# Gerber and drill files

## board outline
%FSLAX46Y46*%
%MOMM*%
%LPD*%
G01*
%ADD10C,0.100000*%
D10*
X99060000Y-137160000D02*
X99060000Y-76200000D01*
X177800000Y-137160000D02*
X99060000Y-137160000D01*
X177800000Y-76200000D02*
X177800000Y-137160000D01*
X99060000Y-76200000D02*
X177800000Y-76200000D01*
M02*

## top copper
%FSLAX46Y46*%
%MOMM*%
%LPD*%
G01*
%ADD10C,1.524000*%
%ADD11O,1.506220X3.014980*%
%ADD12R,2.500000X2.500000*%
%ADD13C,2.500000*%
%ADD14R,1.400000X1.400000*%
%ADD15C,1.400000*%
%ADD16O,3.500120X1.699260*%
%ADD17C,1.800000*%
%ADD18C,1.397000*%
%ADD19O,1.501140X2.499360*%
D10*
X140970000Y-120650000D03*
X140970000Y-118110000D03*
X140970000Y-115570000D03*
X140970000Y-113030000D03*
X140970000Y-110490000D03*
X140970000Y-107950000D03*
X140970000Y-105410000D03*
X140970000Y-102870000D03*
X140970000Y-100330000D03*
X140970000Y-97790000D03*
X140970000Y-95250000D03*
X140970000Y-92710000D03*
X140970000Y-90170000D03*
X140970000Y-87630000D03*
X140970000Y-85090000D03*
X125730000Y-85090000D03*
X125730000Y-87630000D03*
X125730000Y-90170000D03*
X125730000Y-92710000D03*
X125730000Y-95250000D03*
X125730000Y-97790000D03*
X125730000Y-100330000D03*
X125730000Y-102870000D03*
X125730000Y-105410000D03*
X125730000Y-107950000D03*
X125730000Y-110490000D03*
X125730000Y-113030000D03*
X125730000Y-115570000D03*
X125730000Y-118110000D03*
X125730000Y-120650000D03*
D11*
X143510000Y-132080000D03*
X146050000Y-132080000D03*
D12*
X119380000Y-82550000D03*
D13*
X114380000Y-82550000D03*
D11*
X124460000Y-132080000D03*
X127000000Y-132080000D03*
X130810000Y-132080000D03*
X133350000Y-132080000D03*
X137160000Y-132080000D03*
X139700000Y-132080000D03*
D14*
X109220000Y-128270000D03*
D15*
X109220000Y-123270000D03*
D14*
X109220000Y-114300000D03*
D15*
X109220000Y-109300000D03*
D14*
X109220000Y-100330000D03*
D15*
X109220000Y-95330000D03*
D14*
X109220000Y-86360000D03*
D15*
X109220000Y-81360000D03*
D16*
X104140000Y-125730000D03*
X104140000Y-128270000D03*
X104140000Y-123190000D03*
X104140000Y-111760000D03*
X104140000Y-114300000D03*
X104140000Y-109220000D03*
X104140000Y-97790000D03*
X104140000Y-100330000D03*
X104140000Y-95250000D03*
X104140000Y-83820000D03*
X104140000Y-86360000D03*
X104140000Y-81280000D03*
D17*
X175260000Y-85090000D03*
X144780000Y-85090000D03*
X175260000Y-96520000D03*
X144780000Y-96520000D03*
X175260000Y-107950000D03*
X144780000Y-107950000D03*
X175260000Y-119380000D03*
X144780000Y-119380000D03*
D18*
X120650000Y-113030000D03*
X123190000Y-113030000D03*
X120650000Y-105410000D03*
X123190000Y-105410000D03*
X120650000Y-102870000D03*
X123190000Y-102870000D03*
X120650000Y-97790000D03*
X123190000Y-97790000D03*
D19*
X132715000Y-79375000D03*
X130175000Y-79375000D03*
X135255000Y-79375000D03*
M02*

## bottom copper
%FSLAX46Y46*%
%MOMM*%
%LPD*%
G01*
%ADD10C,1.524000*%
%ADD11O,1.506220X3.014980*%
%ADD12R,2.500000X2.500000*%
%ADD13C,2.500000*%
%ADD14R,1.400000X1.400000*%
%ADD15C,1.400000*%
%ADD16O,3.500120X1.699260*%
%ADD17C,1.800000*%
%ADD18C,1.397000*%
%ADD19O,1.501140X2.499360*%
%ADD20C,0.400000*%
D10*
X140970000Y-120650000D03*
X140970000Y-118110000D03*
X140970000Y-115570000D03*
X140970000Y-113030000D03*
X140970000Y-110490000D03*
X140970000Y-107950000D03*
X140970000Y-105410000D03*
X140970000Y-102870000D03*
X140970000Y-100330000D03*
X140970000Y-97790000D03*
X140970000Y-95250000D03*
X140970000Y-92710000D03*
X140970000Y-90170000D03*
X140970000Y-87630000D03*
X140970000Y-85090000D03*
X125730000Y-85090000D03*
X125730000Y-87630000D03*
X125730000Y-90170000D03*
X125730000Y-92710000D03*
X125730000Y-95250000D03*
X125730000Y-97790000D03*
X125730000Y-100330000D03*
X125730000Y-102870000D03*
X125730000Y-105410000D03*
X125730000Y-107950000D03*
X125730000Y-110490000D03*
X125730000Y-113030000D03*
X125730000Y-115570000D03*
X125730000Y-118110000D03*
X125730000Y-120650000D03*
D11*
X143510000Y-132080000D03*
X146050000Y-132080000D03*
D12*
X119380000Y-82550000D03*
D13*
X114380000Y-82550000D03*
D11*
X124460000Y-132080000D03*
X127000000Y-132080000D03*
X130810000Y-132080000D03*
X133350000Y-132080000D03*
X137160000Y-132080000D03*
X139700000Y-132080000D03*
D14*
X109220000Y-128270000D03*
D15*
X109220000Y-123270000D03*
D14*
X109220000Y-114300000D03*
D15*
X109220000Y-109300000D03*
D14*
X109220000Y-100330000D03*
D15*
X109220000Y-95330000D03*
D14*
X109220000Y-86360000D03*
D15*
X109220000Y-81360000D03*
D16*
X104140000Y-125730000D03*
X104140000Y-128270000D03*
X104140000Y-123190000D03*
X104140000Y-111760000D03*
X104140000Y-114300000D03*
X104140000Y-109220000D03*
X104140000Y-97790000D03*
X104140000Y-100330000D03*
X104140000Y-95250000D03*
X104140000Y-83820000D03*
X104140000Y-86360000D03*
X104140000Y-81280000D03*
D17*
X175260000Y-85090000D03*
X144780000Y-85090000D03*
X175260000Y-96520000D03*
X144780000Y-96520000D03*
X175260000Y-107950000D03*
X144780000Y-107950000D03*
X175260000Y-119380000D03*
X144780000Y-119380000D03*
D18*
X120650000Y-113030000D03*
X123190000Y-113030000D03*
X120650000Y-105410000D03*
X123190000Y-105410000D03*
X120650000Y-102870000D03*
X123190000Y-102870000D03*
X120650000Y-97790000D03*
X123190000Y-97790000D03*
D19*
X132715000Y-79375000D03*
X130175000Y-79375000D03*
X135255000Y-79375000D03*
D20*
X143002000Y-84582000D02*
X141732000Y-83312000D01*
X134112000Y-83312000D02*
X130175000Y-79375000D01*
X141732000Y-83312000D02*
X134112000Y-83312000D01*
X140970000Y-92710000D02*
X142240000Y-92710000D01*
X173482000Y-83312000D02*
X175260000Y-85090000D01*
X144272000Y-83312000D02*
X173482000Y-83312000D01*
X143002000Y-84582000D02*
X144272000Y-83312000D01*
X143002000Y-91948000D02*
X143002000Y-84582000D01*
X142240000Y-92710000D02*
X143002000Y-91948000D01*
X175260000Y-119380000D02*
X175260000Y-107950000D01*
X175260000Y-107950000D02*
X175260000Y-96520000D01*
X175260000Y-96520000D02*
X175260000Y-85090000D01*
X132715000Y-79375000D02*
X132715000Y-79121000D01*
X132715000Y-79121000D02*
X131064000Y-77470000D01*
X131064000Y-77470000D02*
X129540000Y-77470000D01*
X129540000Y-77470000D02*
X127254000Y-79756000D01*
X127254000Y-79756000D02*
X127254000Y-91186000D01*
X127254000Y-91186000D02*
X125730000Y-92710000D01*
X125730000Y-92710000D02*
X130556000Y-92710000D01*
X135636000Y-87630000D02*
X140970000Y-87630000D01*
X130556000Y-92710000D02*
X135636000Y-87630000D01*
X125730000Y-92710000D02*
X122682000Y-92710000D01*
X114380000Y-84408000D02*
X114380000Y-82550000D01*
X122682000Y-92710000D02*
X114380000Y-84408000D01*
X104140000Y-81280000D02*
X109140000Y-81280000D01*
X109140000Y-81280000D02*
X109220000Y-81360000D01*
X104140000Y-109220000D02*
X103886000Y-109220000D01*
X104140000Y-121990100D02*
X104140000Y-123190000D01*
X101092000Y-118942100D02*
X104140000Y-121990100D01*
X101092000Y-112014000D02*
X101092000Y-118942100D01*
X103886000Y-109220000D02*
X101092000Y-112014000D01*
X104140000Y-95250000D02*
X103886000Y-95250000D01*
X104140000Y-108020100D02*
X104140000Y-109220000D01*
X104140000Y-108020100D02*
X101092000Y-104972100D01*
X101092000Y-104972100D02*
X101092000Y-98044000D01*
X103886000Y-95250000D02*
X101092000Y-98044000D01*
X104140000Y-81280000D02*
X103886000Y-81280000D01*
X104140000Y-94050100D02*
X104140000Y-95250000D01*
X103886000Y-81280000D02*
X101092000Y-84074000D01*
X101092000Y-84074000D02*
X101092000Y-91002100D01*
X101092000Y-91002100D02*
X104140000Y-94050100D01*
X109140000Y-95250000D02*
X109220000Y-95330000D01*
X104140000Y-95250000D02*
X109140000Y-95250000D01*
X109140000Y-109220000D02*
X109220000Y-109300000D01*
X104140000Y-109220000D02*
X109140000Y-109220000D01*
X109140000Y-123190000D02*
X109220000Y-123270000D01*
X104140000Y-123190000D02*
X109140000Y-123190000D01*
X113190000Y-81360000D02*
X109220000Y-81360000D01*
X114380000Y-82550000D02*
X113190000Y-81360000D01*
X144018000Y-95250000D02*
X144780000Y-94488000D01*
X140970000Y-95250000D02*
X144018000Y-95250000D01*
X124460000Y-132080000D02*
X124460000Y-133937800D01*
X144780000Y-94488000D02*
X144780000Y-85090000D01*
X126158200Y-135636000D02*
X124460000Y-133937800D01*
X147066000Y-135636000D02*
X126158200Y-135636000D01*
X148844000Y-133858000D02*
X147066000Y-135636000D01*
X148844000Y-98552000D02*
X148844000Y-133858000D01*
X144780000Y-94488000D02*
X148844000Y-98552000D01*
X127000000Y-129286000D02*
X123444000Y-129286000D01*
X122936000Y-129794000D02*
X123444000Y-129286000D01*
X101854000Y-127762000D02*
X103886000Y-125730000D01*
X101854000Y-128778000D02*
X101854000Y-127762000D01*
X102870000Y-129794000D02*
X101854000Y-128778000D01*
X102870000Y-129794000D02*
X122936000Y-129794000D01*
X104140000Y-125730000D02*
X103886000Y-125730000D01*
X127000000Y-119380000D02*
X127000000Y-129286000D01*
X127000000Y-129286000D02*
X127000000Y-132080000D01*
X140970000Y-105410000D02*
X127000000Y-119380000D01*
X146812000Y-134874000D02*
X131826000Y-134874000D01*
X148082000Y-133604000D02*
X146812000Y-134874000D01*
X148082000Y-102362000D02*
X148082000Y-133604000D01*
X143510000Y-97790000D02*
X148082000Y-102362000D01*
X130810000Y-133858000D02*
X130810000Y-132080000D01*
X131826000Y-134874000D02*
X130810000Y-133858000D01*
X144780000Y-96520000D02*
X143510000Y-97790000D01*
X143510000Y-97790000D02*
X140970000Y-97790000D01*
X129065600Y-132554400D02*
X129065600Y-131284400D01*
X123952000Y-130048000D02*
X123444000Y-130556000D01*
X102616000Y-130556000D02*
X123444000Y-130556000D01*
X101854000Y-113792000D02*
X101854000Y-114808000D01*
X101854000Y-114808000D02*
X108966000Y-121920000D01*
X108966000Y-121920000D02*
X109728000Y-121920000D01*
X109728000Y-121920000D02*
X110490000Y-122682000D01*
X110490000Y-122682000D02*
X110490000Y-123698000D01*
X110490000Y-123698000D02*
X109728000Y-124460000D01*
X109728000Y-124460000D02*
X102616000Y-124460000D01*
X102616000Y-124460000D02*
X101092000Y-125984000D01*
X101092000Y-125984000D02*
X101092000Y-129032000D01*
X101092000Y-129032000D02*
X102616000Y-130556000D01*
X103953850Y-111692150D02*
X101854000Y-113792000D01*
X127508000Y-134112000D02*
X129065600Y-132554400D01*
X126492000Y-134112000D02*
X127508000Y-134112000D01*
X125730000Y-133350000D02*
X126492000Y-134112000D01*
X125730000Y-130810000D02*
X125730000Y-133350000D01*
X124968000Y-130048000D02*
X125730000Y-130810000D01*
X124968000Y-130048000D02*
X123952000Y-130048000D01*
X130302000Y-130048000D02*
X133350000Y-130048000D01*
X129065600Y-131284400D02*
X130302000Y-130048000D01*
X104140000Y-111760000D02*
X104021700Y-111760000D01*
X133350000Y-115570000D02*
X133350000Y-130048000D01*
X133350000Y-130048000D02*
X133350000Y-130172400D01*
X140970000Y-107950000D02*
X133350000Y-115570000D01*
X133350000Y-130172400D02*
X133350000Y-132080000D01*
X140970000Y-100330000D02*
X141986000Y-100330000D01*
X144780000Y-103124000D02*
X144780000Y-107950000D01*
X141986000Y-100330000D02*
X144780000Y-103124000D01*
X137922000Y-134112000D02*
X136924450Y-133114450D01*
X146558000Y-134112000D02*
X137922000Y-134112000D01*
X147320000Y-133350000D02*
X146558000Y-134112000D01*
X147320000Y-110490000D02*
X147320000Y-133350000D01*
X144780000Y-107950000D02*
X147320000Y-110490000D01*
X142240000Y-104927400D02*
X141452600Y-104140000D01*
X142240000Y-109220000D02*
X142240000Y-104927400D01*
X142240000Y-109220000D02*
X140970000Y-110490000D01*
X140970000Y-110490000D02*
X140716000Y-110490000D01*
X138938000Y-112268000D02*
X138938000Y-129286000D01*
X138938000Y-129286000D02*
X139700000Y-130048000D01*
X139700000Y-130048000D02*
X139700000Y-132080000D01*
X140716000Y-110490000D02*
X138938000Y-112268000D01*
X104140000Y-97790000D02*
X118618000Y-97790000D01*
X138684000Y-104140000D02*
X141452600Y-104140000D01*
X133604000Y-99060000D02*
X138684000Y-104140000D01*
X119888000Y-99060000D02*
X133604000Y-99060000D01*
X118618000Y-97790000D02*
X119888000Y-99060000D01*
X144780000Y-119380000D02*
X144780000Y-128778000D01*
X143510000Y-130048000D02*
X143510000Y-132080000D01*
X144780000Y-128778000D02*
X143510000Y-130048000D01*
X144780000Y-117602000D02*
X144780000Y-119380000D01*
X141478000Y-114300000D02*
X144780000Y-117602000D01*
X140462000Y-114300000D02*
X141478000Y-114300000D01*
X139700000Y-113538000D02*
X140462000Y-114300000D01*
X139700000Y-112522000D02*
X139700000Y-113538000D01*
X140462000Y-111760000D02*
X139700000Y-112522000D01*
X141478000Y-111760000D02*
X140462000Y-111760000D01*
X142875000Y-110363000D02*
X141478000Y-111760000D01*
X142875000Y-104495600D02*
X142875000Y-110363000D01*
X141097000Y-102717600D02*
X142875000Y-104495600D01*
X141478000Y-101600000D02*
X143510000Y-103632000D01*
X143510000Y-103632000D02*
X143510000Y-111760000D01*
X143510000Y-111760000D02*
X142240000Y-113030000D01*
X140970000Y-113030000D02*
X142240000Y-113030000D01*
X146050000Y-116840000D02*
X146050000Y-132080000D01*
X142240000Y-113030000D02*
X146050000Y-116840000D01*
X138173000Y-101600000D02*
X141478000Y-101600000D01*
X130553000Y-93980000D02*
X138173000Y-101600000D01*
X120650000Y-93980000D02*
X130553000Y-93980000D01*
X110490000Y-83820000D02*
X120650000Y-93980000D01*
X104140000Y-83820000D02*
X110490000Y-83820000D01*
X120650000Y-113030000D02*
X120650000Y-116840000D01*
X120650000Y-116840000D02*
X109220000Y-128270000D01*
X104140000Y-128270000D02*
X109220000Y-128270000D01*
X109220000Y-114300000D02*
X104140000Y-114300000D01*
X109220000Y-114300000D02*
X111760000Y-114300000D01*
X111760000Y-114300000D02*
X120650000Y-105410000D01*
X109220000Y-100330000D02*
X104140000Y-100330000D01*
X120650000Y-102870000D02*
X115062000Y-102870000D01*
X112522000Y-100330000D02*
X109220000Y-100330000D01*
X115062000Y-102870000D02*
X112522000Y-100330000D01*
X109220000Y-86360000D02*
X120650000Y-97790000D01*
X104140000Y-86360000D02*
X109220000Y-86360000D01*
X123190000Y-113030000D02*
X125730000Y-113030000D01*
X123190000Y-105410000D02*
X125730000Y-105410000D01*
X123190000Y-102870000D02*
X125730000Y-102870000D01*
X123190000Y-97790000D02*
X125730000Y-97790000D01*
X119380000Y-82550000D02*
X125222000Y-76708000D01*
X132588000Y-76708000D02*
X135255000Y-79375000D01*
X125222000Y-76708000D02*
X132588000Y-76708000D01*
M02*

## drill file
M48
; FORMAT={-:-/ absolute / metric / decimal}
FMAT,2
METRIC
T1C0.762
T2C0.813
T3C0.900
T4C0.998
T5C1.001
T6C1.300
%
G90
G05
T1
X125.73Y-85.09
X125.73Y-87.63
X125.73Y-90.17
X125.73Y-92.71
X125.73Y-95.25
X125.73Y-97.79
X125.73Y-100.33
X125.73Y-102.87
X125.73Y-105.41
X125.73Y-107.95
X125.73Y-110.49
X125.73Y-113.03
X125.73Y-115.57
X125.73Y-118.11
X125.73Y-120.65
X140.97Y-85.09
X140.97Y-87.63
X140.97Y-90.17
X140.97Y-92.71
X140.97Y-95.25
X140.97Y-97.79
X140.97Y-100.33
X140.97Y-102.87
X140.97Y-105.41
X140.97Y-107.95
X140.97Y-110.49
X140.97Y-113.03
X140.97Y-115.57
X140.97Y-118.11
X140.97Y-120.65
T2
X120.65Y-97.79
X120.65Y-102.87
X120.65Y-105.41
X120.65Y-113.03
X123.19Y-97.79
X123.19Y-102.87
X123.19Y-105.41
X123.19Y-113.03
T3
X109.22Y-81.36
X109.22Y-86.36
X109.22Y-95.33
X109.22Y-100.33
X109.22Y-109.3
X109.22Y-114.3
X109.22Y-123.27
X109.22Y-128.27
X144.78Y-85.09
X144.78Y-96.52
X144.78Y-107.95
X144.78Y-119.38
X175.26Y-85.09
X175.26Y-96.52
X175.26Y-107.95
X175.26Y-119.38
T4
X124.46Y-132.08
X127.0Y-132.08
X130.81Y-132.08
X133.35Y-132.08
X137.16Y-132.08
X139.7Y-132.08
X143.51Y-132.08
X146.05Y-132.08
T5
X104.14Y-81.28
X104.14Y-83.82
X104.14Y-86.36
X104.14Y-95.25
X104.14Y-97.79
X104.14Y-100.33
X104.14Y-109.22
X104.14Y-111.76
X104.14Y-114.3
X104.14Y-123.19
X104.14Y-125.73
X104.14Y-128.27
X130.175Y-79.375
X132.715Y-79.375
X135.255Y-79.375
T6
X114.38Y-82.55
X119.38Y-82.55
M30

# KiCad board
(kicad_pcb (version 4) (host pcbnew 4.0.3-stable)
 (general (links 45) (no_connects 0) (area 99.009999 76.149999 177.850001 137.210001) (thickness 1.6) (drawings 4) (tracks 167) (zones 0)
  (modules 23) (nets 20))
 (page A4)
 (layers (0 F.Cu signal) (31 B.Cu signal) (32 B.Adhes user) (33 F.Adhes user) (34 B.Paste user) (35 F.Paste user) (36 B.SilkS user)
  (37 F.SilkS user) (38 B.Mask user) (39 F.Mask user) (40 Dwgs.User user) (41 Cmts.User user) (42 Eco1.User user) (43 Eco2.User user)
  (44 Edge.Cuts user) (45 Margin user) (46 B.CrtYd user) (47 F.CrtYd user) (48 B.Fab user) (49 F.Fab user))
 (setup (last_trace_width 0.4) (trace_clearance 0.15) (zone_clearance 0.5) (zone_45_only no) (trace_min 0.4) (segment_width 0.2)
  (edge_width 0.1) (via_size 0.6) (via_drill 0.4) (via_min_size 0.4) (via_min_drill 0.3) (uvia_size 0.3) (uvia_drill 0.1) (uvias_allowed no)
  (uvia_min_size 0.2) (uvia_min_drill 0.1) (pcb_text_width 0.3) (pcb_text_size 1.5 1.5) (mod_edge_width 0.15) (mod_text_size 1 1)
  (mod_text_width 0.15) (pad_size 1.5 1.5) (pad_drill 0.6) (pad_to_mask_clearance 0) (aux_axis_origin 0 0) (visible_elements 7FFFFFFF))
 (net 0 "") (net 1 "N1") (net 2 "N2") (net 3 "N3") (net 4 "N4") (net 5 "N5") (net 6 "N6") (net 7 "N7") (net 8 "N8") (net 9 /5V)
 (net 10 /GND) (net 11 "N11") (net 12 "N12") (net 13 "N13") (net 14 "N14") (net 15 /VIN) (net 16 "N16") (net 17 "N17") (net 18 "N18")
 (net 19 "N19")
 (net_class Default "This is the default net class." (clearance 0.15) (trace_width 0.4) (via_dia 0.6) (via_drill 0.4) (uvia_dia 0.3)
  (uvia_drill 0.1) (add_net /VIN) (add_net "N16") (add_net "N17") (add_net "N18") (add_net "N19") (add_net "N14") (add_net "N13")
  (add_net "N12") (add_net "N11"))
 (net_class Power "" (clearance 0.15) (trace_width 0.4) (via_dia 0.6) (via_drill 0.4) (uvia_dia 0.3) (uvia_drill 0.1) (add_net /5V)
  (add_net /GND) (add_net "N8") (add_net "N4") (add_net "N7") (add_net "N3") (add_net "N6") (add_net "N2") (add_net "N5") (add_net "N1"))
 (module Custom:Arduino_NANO (layer F.Cu) (at 140.97 120.65 90)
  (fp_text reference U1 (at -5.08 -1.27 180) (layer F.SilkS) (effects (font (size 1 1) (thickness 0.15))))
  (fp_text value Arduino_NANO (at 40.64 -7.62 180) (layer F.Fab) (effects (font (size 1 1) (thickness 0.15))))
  (pad 1 thru_hole circle (at 0 0 90) (size 1.524 1.524) (drill 0.762) (layers *.Cu *.Mask))
  (pad 2 thru_hole circle (at 2.54 0 90) (size 1.524 1.524) (drill 0.762) (layers *.Cu *.Mask))
  (pad 3 thru_hole circle (at 5.08 0 90) (size 1.524 1.524) (drill 0.762) (layers *.Cu *.Mask))
  (pad 4 thru_hole circle (at 7.62 0 90) (size 1.524 1.524) (drill 0.762) (layers *.Cu *.Mask) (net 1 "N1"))
  (pad 5 thru_hole circle (at 10.16 0 90) (size 1.524 1.524) (drill 0.762) (layers *.Cu *.Mask) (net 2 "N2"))
  (pad 6 thru_hole circle (at 12.7 0 90) (size 1.524 1.524) (drill 0.762) (layers *.Cu *.Mask) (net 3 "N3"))
  (pad 7 thru_hole circle (at 15.24 0 90) (size 1.524 1.524) (drill 0.762) (layers *.Cu *.Mask) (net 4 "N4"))
  (pad 8 thru_hole circle (at 17.78 0 90) (size 1.524 1.524) (drill 0.762) (layers *.Cu *.Mask) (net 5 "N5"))
  (pad 9 thru_hole circle (at 20.32 0 90) (size 1.524 1.524) (drill 0.762) (layers *.Cu *.Mask) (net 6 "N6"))
  (pad 10 thru_hole circle (at 22.86 0 90) (size 1.524 1.524) (drill 0.762) (layers *.Cu *.Mask) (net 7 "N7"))
  (pad 11 thru_hole circle (at 25.4 0 90) (size 1.524 1.524) (drill 0.762) (layers *.Cu *.Mask) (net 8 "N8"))
  (pad 12 thru_hole circle (at 27.94 0 90) (size 1.524 1.524) (drill 0.762) (layers *.Cu *.Mask) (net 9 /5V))
  (pad 13 thru_hole circle (at 30.48 0 90) (size 1.524 1.524) (drill 0.762) (layers *.Cu *.Mask))
  (pad 14 thru_hole circle (at 33.02 0 90) (size 1.524 1.524) (drill 0.762) (layers *.Cu *.Mask) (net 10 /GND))
  (pad 15 thru_hole circle (at 35.56 0 90) (size 1.524 1.524) (drill 0.762) (layers *.Cu *.Mask))
  (pad 16 thru_hole circle (at 35.56 -15.24 90) (size 1.524 1.524) (drill 0.762) (layers *.Cu *.Mask))
  (pad 17 thru_hole circle (at 33.02 -15.24 90) (size 1.524 1.524) (drill 0.762) (layers *.Cu *.Mask))
  (pad 18 thru_hole circle (at 30.48 -15.24 90) (size 1.524 1.524) (drill 0.762) (layers *.Cu *.Mask))
  (pad 19 thru_hole circle (at 27.94 -15.24 90) (size 1.524 1.524) (drill 0.762) (layers *.Cu *.Mask) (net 10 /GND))
  (pad 20 thru_hole circle (at 25.4 -15.24 90) (size 1.524 1.524) (drill 0.762) (layers *.Cu *.Mask))
  (pad 21 thru_hole circle (at 22.86 -15.24 90) (size 1.524 1.524) (drill 0.762) (layers *.Cu *.Mask) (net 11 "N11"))
  (pad 22 thru_hole circle (at 20.32 -15.24 90) (size 1.524 1.524) (drill 0.762) (layers *.Cu *.Mask))
  (pad 23 thru_hole circle (at 17.78 -15.24 90) (size 1.524 1.524) (drill 0.762) (layers *.Cu *.Mask) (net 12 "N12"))
  (pad 24 thru_hole circle (at 15.24 -15.24 90) (size 1.524 1.524) (drill 0.762) (layers *.Cu *.Mask) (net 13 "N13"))
  (pad 25 thru_hole circle (at 12.7 -15.24 90) (size 1.524 1.524) (drill 0.762) (layers *.Cu *.Mask))
  (pad 26 thru_hole circle (at 10.16 -15.24 90) (size 1.524 1.524) (drill 0.762) (layers *.Cu *.Mask))
  (pad 27 thru_hole circle (at 7.62 -15.24 90) (size 1.524 1.524) (drill 0.762) (layers *.Cu *.Mask) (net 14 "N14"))
  (pad 28 thru_hole circle (at 5.08 -15.24 90) (size 1.524 1.524) (drill 0.762) (layers *.Cu *.Mask))
  (pad 29 thru_hole circle (at 2.54 -15.24 90) (size 1.524 1.524) (drill 0.762) (layers *.Cu *.Mask))
  (pad 30 thru_hole circle (at 0 -15.24 90) (size 1.524 1.524) (drill 0.762) (layers *.Cu *.Mask)))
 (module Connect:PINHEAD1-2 (layer F.Cu) (at 144.78 132.08)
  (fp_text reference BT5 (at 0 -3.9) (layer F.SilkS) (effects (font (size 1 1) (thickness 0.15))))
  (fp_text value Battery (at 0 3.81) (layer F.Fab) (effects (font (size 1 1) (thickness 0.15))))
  (pad 1 thru_hole oval (at -1.27 0) (size 1.50622 3.01498) (drill 0.99822) (layers *.Cu *.Mask) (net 5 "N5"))
  (pad 2 thru_hole oval (at 1.27 0) (size 1.50622 3.01498) (drill 0.99822) (layers *.Cu *.Mask) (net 1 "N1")))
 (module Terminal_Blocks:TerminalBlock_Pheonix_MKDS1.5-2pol (layer F.Cu) (at 119.38 82.55 180)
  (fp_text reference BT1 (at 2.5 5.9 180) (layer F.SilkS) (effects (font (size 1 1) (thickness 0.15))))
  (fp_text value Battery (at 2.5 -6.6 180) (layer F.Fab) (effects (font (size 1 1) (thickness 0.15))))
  (pad 1 thru_hole rect (at 0 0 180) (size 2.5 2.5) (drill 1.3) (layers *.Cu *.Mask F.SilkS) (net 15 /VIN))
  (pad 2 thru_hole circle (at 5 0 180) (size 2.5 2.5) (drill 1.3) (layers *.Cu *.Mask F.SilkS) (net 10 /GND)))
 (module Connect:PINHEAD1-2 (layer F.Cu) (at 125.73 132.08)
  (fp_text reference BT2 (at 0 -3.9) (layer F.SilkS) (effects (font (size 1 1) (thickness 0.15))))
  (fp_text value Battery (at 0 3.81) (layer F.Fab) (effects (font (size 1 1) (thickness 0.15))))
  (pad 1 thru_hole oval (at -1.27 0) (size 1.50622 3.01498) (drill 0.99822) (layers *.Cu *.Mask) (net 8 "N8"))
  (pad 2 thru_hole oval (at 1.27 0) (size 1.50622 3.01498) (drill 0.99822) (layers *.Cu *.Mask) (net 4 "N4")))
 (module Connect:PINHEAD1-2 (layer F.Cu) (at 132.08 132.08)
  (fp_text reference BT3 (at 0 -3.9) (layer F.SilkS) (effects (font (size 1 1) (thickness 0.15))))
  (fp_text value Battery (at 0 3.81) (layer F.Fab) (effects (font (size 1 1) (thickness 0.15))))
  (pad 1 thru_hole oval (at -1.27 0) (size 1.50622 3.01498) (drill 0.99822) (layers *.Cu *.Mask) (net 7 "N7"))
  (pad 2 thru_hole oval (at 1.27 0) (size 1.50622 3.01498) (drill 0.99822) (layers *.Cu *.Mask) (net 3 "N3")))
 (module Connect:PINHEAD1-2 (layer F.Cu) (at 138.43 132.08)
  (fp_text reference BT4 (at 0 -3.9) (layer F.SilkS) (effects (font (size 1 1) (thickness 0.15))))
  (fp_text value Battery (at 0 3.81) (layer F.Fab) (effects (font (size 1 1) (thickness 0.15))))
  (pad 1 thru_hole oval (at -1.27 0) (size 1.50622 3.01498) (drill 0.99822) (layers *.Cu *.Mask) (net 6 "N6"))
  (pad 2 thru_hole oval (at 1.27 0) (size 1.50622 3.01498) (drill 0.99822) (layers *.Cu *.Mask) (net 2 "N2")))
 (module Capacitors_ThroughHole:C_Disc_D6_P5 (layer F.Cu) (at 109.22 128.27 90)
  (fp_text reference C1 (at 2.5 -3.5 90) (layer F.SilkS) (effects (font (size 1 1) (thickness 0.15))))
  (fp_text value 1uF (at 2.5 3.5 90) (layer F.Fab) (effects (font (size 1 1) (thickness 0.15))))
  (pad 1 thru_hole rect (at 0 0 90) (size 1.4 1.4) (drill 0.9) (layers *.Cu *.Mask F.SilkS) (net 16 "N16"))
  (pad 2 thru_hole circle (at 5 0 90) (size 1.4 1.4) (drill 0.9) (layers *.Cu *.Mask F.SilkS) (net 10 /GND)))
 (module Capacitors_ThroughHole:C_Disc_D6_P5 (layer F.Cu) (at 109.22 114.3 90)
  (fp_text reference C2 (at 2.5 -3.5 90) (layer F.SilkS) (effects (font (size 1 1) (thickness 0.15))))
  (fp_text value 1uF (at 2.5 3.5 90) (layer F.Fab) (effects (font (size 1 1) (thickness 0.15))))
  (pad 1 thru_hole rect (at 0 0 90) (size 1.4 1.4) (drill 0.9) (layers *.Cu *.Mask F.SilkS) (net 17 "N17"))
  (pad 2 thru_hole circle (at 5 0 90) (size 1.4 1.4) (drill 0.9) (layers *.Cu *.Mask F.SilkS) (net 10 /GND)))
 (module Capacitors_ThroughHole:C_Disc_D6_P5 (layer F.Cu) (at 109.22 100.33 90)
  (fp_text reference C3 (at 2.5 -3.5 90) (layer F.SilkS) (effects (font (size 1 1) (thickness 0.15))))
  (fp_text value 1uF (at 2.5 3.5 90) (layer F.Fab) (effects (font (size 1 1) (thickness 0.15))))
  (pad 1 thru_hole rect (at 0 0 90) (size 1.4 1.4) (drill 0.9) (layers *.Cu *.Mask F.SilkS) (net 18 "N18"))
  (pad 2 thru_hole circle (at 5 0 90) (size 1.4 1.4) (drill 0.9) (layers *.Cu *.Mask F.SilkS) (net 10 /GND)))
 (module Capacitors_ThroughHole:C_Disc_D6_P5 (layer F.Cu) (at 109.22 86.36 90)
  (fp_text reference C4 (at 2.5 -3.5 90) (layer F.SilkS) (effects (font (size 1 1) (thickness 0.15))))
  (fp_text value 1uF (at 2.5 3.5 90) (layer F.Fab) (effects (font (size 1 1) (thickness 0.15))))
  (pad 1 thru_hole rect (at 0 0 90) (size 1.4 1.4) (drill 0.9) (layers *.Cu *.Mask F.SilkS) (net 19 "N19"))
  (pad 2 thru_hole circle (at 5 0 90) (size 1.4 1.4) (drill 0.9) (layers *.Cu *.Mask F.SilkS) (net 10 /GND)))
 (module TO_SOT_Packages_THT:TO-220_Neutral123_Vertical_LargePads (layer F.Cu) (at 104.14 125.73 90)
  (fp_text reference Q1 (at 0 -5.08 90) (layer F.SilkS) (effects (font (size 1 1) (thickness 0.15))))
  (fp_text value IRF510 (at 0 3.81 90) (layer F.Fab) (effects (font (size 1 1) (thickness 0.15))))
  (pad 2 thru_hole oval (at 0 0 180) (size 3.50012 1.69926) (drill 1.00076) (layers *.Cu *.Mask F.SilkS) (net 4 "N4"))
  (pad 1 thru_hole oval (at -2.54 0 180) (size 3.50012 1.69926) (drill 1.00076) (layers *.Cu *.Mask F.SilkS) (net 16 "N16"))
  (pad 3 thru_hole oval (at 2.54 0 180) (size 3.50012 1.69926) (drill 1.00076) (layers *.Cu *.Mask F.SilkS) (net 10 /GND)))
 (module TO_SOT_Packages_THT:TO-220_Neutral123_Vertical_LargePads (layer F.Cu) (at 104.14 111.76 90)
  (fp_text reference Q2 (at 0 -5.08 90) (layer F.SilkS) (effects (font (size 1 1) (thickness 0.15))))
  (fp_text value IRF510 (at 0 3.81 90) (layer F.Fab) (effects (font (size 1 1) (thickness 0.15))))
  (pad 2 thru_hole oval (at 0 0 180) (size 3.50012 1.69926) (drill 1.00076) (layers *.Cu *.Mask F.SilkS) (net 3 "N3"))
  (pad 1 thru_hole oval (at -2.54 0 180) (size 3.50012 1.69926) (drill 1.00076) (layers *.Cu *.Mask F.SilkS) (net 17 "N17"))
  (pad 3 thru_hole oval (at 2.54 0 180) (size 3.50012 1.69926) (drill 1.00076) (layers *.Cu *.Mask F.SilkS) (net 10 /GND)))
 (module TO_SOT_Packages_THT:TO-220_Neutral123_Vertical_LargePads (layer F.Cu) (at 104.14 97.79 90)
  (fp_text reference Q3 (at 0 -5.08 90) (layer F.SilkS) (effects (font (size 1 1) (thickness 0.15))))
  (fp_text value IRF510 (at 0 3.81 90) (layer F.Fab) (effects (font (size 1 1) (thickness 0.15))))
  (pad 2 thru_hole oval (at 0 0 180) (size 3.50012 1.69926) (drill 1.00076) (layers *.Cu *.Mask F.SilkS) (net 2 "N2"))
  (pad 1 thru_hole oval (at -2.54 0 180) (size 3.50012 1.69926) (drill 1.00076) (layers *.Cu *.Mask F.SilkS) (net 18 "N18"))
  (pad 3 thru_hole oval (at 2.54 0 180) (size 3.50012 1.69926) (drill 1.00076) (layers *.Cu *.Mask F.SilkS) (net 10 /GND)))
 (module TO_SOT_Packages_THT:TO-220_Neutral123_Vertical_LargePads (layer F.Cu) (at 104.14 83.82 90)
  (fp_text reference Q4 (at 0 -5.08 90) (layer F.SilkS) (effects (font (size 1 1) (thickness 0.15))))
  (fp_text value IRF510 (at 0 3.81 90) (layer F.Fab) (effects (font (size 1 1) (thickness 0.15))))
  (pad 2 thru_hole oval (at 0 0 180) (size 3.50012 1.69926) (drill 1.00076) (layers *.Cu *.Mask F.SilkS) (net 1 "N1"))
  (pad 1 thru_hole oval (at -2.54 0 180) (size 3.50012 1.69926) (drill 1.00076) (layers *.Cu *.Mask F.SilkS) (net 19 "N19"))
  (pad 3 thru_hole oval (at 2.54 0 180) (size 3.50012 1.69926) (drill 1.00076) (layers *.Cu *.Mask F.SilkS) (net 10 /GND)))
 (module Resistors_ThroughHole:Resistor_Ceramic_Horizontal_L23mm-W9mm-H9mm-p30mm (layer F.Cu) (at 160.02 85.09 180)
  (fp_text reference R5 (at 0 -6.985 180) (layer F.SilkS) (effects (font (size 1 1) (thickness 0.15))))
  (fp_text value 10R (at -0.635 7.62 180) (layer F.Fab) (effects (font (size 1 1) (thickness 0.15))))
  (pad 1 thru_hole circle (at -15.24 0) (size 1.8 1.8) (drill 0.9) (layers *.Cu *.Mask F.SilkS) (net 9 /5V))
  (pad 2 thru_hole circle (at 15.24 0) (size 1.8 1.8) (drill 0.9) (layers *.Cu *.Mask F.SilkS) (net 8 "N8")))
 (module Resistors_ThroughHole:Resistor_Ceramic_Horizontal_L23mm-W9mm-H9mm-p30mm (layer F.Cu) (at 160.02 96.52 180)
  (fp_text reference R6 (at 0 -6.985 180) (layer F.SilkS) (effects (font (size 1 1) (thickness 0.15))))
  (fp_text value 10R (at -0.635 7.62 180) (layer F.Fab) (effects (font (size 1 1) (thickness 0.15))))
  (pad 1 thru_hole circle (at -15.24 0) (size 1.8 1.8) (drill 0.9) (layers *.Cu *.Mask F.SilkS) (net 9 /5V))
  (pad 2 thru_hole circle (at 15.24 0) (size 1.8 1.8) (drill 0.9) (layers *.Cu *.Mask F.SilkS) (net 7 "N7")))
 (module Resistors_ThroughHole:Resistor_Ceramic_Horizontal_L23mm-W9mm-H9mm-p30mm (layer F.Cu) (at 160.02 107.95 180)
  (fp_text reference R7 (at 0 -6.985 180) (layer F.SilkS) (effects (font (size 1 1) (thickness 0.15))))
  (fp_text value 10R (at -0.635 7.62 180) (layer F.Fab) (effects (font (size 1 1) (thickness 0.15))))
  (pad 1 thru_hole circle (at -15.24 0) (size 1.8 1.8) (drill 0.9) (layers *.Cu *.Mask F.SilkS) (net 9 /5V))
  (pad 2 thru_hole circle (at 15.24 0) (size 1.8 1.8) (drill 0.9) (layers *.Cu *.Mask F.SilkS) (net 6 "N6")))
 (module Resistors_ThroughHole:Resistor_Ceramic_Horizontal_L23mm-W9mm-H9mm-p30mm (layer F.Cu) (at 160.02 119.38 180)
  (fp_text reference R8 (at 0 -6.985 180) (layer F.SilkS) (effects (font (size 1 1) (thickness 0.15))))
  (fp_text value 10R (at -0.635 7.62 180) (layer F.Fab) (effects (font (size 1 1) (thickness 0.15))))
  (pad 1 thru_hole circle (at -15.24 0) (size 1.8 1.8) (drill 0.9) (layers *.Cu *.Mask F.SilkS) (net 9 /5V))
  (pad 2 thru_hole circle (at 15.24 0) (size 1.8 1.8) (drill 0.9) (layers *.Cu *.Mask F.SilkS) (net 5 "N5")))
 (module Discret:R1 (layer F.Cu) (at 121.92 113.03)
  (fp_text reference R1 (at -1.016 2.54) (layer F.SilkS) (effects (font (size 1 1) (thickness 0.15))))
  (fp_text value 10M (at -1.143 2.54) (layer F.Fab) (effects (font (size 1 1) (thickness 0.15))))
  (pad 1 thru_hole circle (at -1.27 0) (size 1.397 1.397) (drill 0.8128) (layers *.Cu *.Mask F.SilkS) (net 16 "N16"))
  (pad 2 thru_hole circle (at 1.27 0) (size 1.397 1.397) (drill 0.8128) (layers *.Cu *.Mask F.SilkS) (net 14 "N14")))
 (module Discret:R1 (layer F.Cu) (at 121.92 105.41)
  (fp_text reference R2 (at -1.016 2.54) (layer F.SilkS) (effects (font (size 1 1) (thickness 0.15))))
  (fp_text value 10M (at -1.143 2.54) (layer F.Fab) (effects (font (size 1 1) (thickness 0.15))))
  (pad 1 thru_hole circle (at -1.27 0) (size 1.397 1.397) (drill 0.8128) (layers *.Cu *.Mask F.SilkS) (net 17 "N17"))
  (pad 2 thru_hole circle (at 1.27 0) (size 1.397 1.397) (drill 0.8128) (layers *.Cu *.Mask F.SilkS) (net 13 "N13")))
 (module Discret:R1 (layer F.Cu) (at 121.92 102.87)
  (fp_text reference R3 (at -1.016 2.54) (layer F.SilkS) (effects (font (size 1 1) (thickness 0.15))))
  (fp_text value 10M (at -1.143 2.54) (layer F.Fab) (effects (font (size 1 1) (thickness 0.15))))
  (pad 1 thru_hole circle (at -1.27 0) (size 1.397 1.397) (drill 0.8128) (layers *.Cu *.Mask F.SilkS) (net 18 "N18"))
  (pad 2 thru_hole circle (at 1.27 0) (size 1.397 1.397) (drill 0.8128) (layers *.Cu *.Mask F.SilkS) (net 12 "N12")))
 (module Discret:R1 (layer F.Cu) (at 121.92 97.79)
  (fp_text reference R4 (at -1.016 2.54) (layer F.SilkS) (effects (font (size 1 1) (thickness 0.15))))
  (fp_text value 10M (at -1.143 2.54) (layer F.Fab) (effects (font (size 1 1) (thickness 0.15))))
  (pad 1 thru_hole circle (at -1.27 0) (size 1.397 1.397) (drill 0.8128) (layers *.Cu *.Mask F.SilkS) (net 19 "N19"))
  (pad 2 thru_hole circle (at 1.27 0) (size 1.397 1.397) (drill 0.8128) (layers *.Cu *.Mask F.SilkS) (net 11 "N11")))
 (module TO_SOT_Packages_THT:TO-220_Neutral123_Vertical (layer F.Cu) (at 132.715 79.375)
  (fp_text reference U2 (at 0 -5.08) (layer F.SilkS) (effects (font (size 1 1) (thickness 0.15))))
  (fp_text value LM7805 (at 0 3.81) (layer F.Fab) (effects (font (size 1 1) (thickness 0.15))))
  (pad 2 thru_hole oval (at 0 0 90) (size 2.49936 1.50114) (drill 1.00076) (layers *.Cu *.Mask) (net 10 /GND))
  (pad 1 thru_hole oval (at -2.54 0 90) (size 2.49936 1.50114) (drill 1.00076) (layers *.Cu *.Mask) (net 9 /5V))
  (pad 3 thru_hole oval (at 2.54 0 90) (size 2.49936 1.50114) (drill 1.00076) (layers *.Cu *.Mask) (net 15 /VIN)))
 (gr_line (start 99.06 137.16) (end 99.06 76.2) (angle 90) (layer Edge.Cuts) (width 0.1))
 (gr_line (start 177.8 137.16) (end 99.06 137.16) (angle 90) (layer Edge.Cuts) (width 0.1))
 (gr_line (start 177.8 76.2) (end 177.8 137.16) (angle 90) (layer Edge.Cuts) (width 0.1))
 (gr_line (start 99.06 76.2) (end 177.8 76.2) (angle 90) (layer Edge.Cuts) (width 0.1))
 (segment (start 143.002 84.582) (end 141.732 83.312) (width 0.4) (layer B.Cu) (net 9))
 (segment (start 134.112 83.312) (end 130.175 79.375) (width 0.4) (layer B.Cu) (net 9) (status 800000))
 (segment (start 141.732 83.312) (end 134.112 83.312) (width 0.4) (layer B.Cu) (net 9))
 (segment (start 140.97 92.71) (end 142.24 92.71) (width 0.4) (layer B.Cu) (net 9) (status 400000))
 (segment (start 173.482 83.312) (end 175.26 85.09) (width 0.4) (layer B.Cu) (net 9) (status 800000))
 (segment (start 144.272 83.312) (end 173.482 83.312) (width 0.4) (layer B.Cu) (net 9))
 (segment (start 143.002 84.582) (end 144.272 83.312) (width 0.4) (layer B.Cu) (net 9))
 (segment (start 143.002 91.948) (end 143.002 84.582) (width 0.4) (layer B.Cu) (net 9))
 (segment (start 142.24 92.71) (end 143.002 91.948) (width 0.4) (layer B.Cu) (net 9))
 (segment (start 175.26 119.38) (end 175.26 107.95) (width 0.4) (layer B.Cu) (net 9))
 (segment (start 175.26 107.95) (end 175.26 96.52) (width 0.4) (layer B.Cu) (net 9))
 (segment (start 175.26 96.52) (end 175.26 85.09) (width 0.4) (layer B.Cu) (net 9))
 (segment (start 132.715 79.375) (end 132.715 79.121) (width 0.4) (layer B.Cu) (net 10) (status C00000))
 (segment (start 132.715 79.121) (end 131.064 77.47) (width 0.4) (layer B.Cu) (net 10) (status 400000))
 (segment (start 131.064 77.47) (end 129.54 77.47) (width 0.4) (layer B.Cu) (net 10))
 (segment (start 129.54 77.47) (end 127.254 79.756) (width 0.4) (layer B.Cu) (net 10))
 (segment (start 127.254 79.756) (end 127.254 91.186) (width 0.4) (layer B.Cu) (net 10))
 (segment (start 127.254 91.186) (end 125.73 92.71) (width 0.4) (layer B.Cu) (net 10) (status 800000))
 (segment (start 125.73 92.71) (end 130.556 92.71) (width 0.4) (layer B.Cu) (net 10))
 (segment (start 135.636 87.63) (end 140.97 87.63) (width 0.4) (layer B.Cu) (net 10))
 (segment (start 130.556 92.71) (end 135.636 87.63) (width 0.4) (layer B.Cu) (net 10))
 (segment (start 125.73 92.71) (end 122.682 92.71) (width 0.4) (layer B.Cu) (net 10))
 (segment (start 114.38 84.408) (end 114.38 82.55) (width 0.4) (layer B.Cu) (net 10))
 (segment (start 122.682 92.71) (end 114.38 84.408) (width 0.4) (layer B.Cu) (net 10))
 (segment (start 104.14 81.28) (end 109.14 81.28) (width 0.4) (layer B.Cu) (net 10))
 (segment (start 109.14 81.28) (end 109.22 81.36) (width 0.4) (layer B.Cu) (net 10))
 (segment (start 104.14 109.22) (end 103.886 109.22) (width 0.4) (layer B.Cu) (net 10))
 (segment (start 104.14 121.9901) (end 104.14 123.19) (width 0.4) (layer B.Cu) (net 10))
 (segment (start 101.092 118.9421) (end 104.14 121.9901) (width 0.4) (layer B.Cu) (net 10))
 (segment (start 101.092 112.014) (end 101.092 118.9421) (width 0.4) (layer B.Cu) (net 10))
 (segment (start 103.886 109.22) (end 101.092 112.014) (width 0.4) (layer B.Cu) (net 10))
 (segment (start 104.14 95.25) (end 103.886 95.25) (width 0.4) (layer B.Cu) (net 10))
 (segment (start 104.14 108.0201) (end 104.14 109.22) (width 0.4) (layer B.Cu) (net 10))
 (segment (start 104.14 108.0201) (end 101.092 104.9721) (width 0.4) (layer B.Cu) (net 10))
 (segment (start 101.092 104.9721) (end 101.092 98.044) (width 0.4) (layer B.Cu) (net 10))
 (segment (start 103.886 95.25) (end 101.092 98.044) (width 0.4) (layer B.Cu) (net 10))
 (segment (start 104.14 81.28) (end 103.886 81.28) (width 0.4) (layer B.Cu) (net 10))
 (segment (start 104.14 94.0501) (end 104.14 95.25) (width 0.4) (layer B.Cu) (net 10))
 (segment (start 103.886 81.28) (end 101.092 84.074) (width 0.4) (layer B.Cu) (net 10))
 (segment (start 101.092 84.074) (end 101.092 91.0021) (width 0.4) (layer B.Cu) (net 10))
 (segment (start 101.092 91.0021) (end 104.14 94.0501) (width 0.4) (layer B.Cu) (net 10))
 (segment (start 109.14 95.25) (end 109.22 95.33) (width 0.4) (layer B.Cu) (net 10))
 (segment (start 104.14 95.25) (end 109.14 95.25) (width 0.4) (layer B.Cu) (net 10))
 (segment (start 109.14 109.22) (end 109.22 109.3) (width 0.4) (layer B.Cu) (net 10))
 (segment (start 104.14 109.22) (end 109.14 109.22) (width 0.4) (layer B.Cu) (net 10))
 (segment (start 109.14 123.19) (end 109.22 123.27) (width 0.4) (layer B.Cu) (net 10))
 (segment (start 104.14 123.19) (end 109.14 123.19) (width 0.4) (layer B.Cu) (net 10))
 (segment (start 113.19 81.36) (end 109.22 81.36) (width 0.4) (layer B.Cu) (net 10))
 (segment (start 114.38 82.55) (end 113.19 81.36) (width 0.4) (layer B.Cu) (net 10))
 (segment (start 144.018 95.25) (end 144.78 94.488) (width 0.4) (layer B.Cu) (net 8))
 (segment (start 140.97 95.25) (end 144.018 95.25) (width 0.4) (layer B.Cu) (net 8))
 (segment (start 124.46 132.08) (end 124.46 133.9378) (width 0.4) (layer B.Cu) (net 8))
 (segment (start 144.78 94.488) (end 144.78 85.09) (width 0.4) (layer B.Cu) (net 8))
 (segment (start 126.1582 135.636) (end 124.46 133.9378) (width 0.4) (layer B.Cu) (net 8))
 (segment (start 147.066 135.636) (end 126.1582 135.636) (width 0.4) (layer B.Cu) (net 8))
 (segment (start 148.844 133.858) (end 147.066 135.636) (width 0.4) (layer B.Cu) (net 8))
 (segment (start 148.844 98.552) (end 148.844 133.858) (width 0.4) (layer B.Cu) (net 8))
 (segment (start 144.78 94.488) (end 148.844 98.552) (width 0.4) (layer B.Cu) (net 8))
 (segment (start 127 129.286) (end 123.444 129.286) (width 0.4) (layer B.Cu) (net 4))
 (segment (start 122.936 129.794) (end 123.444 129.286) (width 0.4) (layer B.Cu) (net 4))
 (segment (start 101.854 127.762) (end 103.886 125.73) (width 0.4) (layer B.Cu) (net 4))
 (segment (start 101.854 128.778) (end 101.854 127.762) (width 0.4) (layer B.Cu) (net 4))
 (segment (start 102.87 129.794) (end 101.854 128.778) (width 0.4) (layer B.Cu) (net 4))
 (segment (start 102.87 129.794) (end 122.936 129.794) (width 0.4) (layer B.Cu) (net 4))
 (segment (start 104.14 125.73) (end 103.886 125.73) (width 0.4) (layer B.Cu) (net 4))
 (segment (start 127 119.38) (end 127 129.286) (width 0.4) (layer B.Cu) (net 4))
 (segment (start 127 129.286) (end 127 132.08) (width 0.4) (layer B.Cu) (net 4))
 (segment (start 140.97 105.41) (end 127 119.38) (width 0.4) (layer B.Cu) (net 4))
 (segment (start 146.812 134.874) (end 131.826 134.874) (width 0.4) (layer B.Cu) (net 7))
 (segment (start 148.082 133.604) (end 146.812 134.874) (width 0.4) (layer B.Cu) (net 7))
 (segment (start 148.082 102.362) (end 148.082 133.604) (width 0.4) (layer B.Cu) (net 7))
 (segment (start 143.51 97.79) (end 148.082 102.362) (width 0.4) (layer B.Cu) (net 7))
 (segment (start 130.81 133.858) (end 130.81 132.08) (width 0.4) (layer B.Cu) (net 7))
 (segment (start 131.826 134.874) (end 130.81 133.858) (width 0.4) (layer B.Cu) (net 7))
 (segment (start 144.78 96.52) (end 143.51 97.79) (width 0.4) (layer B.Cu) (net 7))
 (segment (start 143.51 97.79) (end 140.97 97.79) (width 0.4) (layer B.Cu) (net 7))
 (segment (start 129.0656 132.5544) (end 129.0656 131.2844) (width 0.4) (layer B.Cu) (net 3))
 (segment (start 123.952 130.048) (end 123.444 130.556) (width 0.4) (layer B.Cu) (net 3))
 (segment (start 102.616 130.556) (end 123.444 130.556) (width 0.4) (layer B.Cu) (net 3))
 (segment (start 101.854 113.792) (end 101.854 114.808) (width 0.4) (layer B.Cu) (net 3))
 (segment (start 101.854 114.808) (end 108.966 121.92) (width 0.4) (layer B.Cu) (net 3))
 (segment (start 108.966 121.92) (end 109.728 121.92) (width 0.4) (layer B.Cu) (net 3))
 (segment (start 109.728 121.92) (end 110.49 122.682) (width 0.4) (layer B.Cu) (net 3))
 (segment (start 110.49 122.682) (end 110.49 123.698) (width 0.4) (layer B.Cu) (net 3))
 (segment (start 110.49 123.698) (end 109.728 124.46) (width 0.4) (layer B.Cu) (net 3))
 (segment (start 109.728 124.46) (end 102.616 124.46) (width 0.4) (layer B.Cu) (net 3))
 (segment (start 102.616 124.46) (end 101.092 125.984) (width 0.4) (layer B.Cu) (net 3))
 (segment (start 101.092 125.984) (end 101.092 129.032) (width 0.4) (layer B.Cu) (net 3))
 (segment (start 101.092 129.032) (end 102.616 130.556) (width 0.4) (layer B.Cu) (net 3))
 (segment (start 103.95385 111.69215) (end 101.854 113.792) (width 0.4) (layer B.Cu) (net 3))
 (segment (start 127.508 134.112) (end 129.0656 132.5544) (width 0.4) (layer B.Cu) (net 3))
 (segment (start 126.492 134.112) (end 127.508 134.112) (width 0.4) (layer B.Cu) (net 3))
 (segment (start 125.73 133.35) (end 126.492 134.112) (width 0.4) (layer B.Cu) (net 3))
 (segment (start 125.73 130.81) (end 125.73 133.35) (width 0.4) (layer B.Cu) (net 3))
 (segment (start 124.968 130.048) (end 125.73 130.81) (width 0.4) (layer B.Cu) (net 3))
 (segment (start 124.968 130.048) (end 123.952 130.048) (width 0.4) (layer B.Cu) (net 3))
 (segment (start 130.302 130.048) (end 133.35 130.048) (width 0.4) (layer B.Cu) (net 3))
 (segment (start 129.0656 131.2844) (end 130.302 130.048) (width 0.4) (layer B.Cu) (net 3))
 (segment (start 104.14 111.76) (end 104.0217 111.76) (width 0.4) (layer B.Cu) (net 3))
 (segment (start 133.35 115.57) (end 133.35 130.048) (width 0.4) (layer B.Cu) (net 3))
 (segment (start 133.35 130.048) (end 133.35 130.1724) (width 0.4) (layer B.Cu) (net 3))
 (segment (start 140.97 107.95) (end 133.35 115.57) (width 0.4) (layer B.Cu) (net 3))
 (segment (start 133.35 130.1724) (end 133.35 132.08) (width 0.4) (layer B.Cu) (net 3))
 (segment (start 140.97 100.33) (end 141.986 100.33) (width 0.4) (layer B.Cu) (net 6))
 (segment (start 144.78 103.124) (end 144.78 107.95) (width 0.4) (layer B.Cu) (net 6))
 (segment (start 141.986 100.33) (end 144.78 103.124) (width 0.4) (layer B.Cu) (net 6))
 (segment (start 137.922 134.112) (end 136.92445 133.11445) (width 0.4) (layer B.Cu) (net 6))
 (segment (start 146.558 134.112) (end 137.922 134.112) (width 0.4) (layer B.Cu) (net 6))
 (segment (start 147.32 133.35) (end 146.558 134.112) (width 0.4) (layer B.Cu) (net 6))
 (segment (start 147.32 110.49) (end 147.32 133.35) (width 0.4) (layer B.Cu) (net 6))
 (segment (start 144.78 107.95) (end 147.32 110.49) (width 0.4) (layer B.Cu) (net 6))
 (segment (start 142.24 104.9274) (end 141.4526 104.14) (width 0.4) (layer B.Cu) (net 2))
 (segment (start 142.24 109.22) (end 142.24 104.9274) (width 0.4) (layer B.Cu) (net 2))
 (segment (start 142.24 109.22) (end 140.97 110.49) (width 0.4) (layer B.Cu) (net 2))
 (segment (start 140.97 110.49) (end 140.716 110.49) (width 0.4) (layer B.Cu) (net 2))
 (segment (start 138.938 112.268) (end 138.938 129.286) (width 0.4) (layer B.Cu) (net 2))
 (segment (start 138.938 129.286) (end 139.7 130.048) (width 0.4) (layer B.Cu) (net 2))
 (segment (start 139.7 130.048) (end 139.7 132.08) (width 0.4) (layer B.Cu) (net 2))
 (segment (start 140.716 110.49) (end 138.938 112.268) (width 0.4) (layer B.Cu) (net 2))
 (segment (start 104.14 97.79) (end 118.618 97.79) (width 0.4) (layer B.Cu) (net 2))
 (segment (start 138.684 104.14) (end 141.4526 104.14) (width 0.4) (layer B.Cu) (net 2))
 (segment (start 133.604 99.06) (end 138.684 104.14) (width 0.4) (layer B.Cu) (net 2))
 (segment (start 119.888 99.06) (end 133.604 99.06) (width 0.4) (layer B.Cu) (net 2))
 (segment (start 118.618 97.79) (end 119.888 99.06) (width 0.4) (layer B.Cu) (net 2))
 (segment (start 144.78 119.38) (end 144.78 128.778) (width 0.4) (layer B.Cu) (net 5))
 (segment (start 143.51 130.048) (end 143.51 132.08) (width 0.4) (layer B.Cu) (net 5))
 (segment (start 144.78 128.778) (end 143.51 130.048) (width 0.4) (layer B.Cu) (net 5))
 (segment (start 144.78 117.602) (end 144.78 119.38) (width 0.4) (layer B.Cu) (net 5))
 (segment (start 141.478 114.3) (end 144.78 117.602) (width 0.4) (layer B.Cu) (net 5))
 (segment (start 140.462 114.3) (end 141.478 114.3) (width 0.4) (layer B.Cu) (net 5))
 (segment (start 139.7 113.538) (end 140.462 114.3) (width 0.4) (layer B.Cu) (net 5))
 (segment (start 139.7 112.522) (end 139.7 113.538) (width 0.4) (layer B.Cu) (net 5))
 (segment (start 140.462 111.76) (end 139.7 112.522) (width 0.4) (layer B.Cu) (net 5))
 (segment (start 141.478 111.76) (end 140.462 111.76) (width 0.4) (layer B.Cu) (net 5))
 (segment (start 142.875 110.363) (end 141.478 111.76) (width 0.4) (layer B.Cu) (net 5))
 (segment (start 142.875 104.4956) (end 142.875 110.363) (width 0.4) (layer B.Cu) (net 5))
 (segment (start 141.097 102.7176) (end 142.875 104.4956) (width 0.4) (layer B.Cu) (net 5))
 (segment (start 141.478 101.6) (end 143.51 103.632) (width 0.4) (layer B.Cu) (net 1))
 (segment (start 143.51 103.632) (end 143.51 111.76) (width 0.4) (layer B.Cu) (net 1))
 (segment (start 143.51 111.76) (end 142.24 113.03) (width 0.4) (layer B.Cu) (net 1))
 (segment (start 140.97 113.03) (end 142.24 113.03) (width 0.4) (layer B.Cu) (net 1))
 (segment (start 146.05 116.84) (end 146.05 132.08) (width 0.4) (layer B.Cu) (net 1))
 (segment (start 142.24 113.03) (end 146.05 116.84) (width 0.4) (layer B.Cu) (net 1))
 (segment (start 138.173 101.6) (end 141.478 101.6) (width 0.4) (layer B.Cu) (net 1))
 (segment (start 130.553 93.98) (end 138.173 101.6) (width 0.4) (layer B.Cu) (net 1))
 (segment (start 120.65 93.98) (end 130.553 93.98) (width 0.4) (layer B.Cu) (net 1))
 (segment (start 110.49 83.82) (end 120.65 93.98) (width 0.4) (layer B.Cu) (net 1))
 (segment (start 104.14 83.82) (end 110.49 83.82) (width 0.4) (layer B.Cu) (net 1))
 (segment (start 120.65 113.03) (end 120.65 116.84) (width 0.4) (layer B.Cu) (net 16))
 (segment (start 120.65 116.84) (end 109.22 128.27) (width 0.4) (layer B.Cu) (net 16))
 (segment (start 104.14 128.27) (end 109.22 128.27) (width 0.4) (layer B.Cu) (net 16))
 (segment (start 109.22 114.3) (end 104.14 114.3) (width 0.4) (layer B.Cu) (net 17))
 (segment (start 109.22 114.3) (end 111.76 114.3) (width 0.4) (layer B.Cu) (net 17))
 (segment (start 111.76 114.3) (end 120.65 105.41) (width 0.4) (layer B.Cu) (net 17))
 (segment (start 109.22 100.33) (end 104.14 100.33) (width 0.4) (layer B.Cu) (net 18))
 (segment (start 120.65 102.87) (end 115.062 102.87) (width 0.4) (layer B.Cu) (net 18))
 (segment (start 112.522 100.33) (end 109.22 100.33) (width 0.4) (layer B.Cu) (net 18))
 (segment (start 115.062 102.87) (end 112.522 100.33) (width 0.4) (layer B.Cu) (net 18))
 (segment (start 109.22 86.36) (end 120.65 97.79) (width 0.4) (layer B.Cu) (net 19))
 (segment (start 104.14 86.36) (end 109.22 86.36) (width 0.4) (layer B.Cu) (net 19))
 (segment (start 123.19 113.03) (end 125.73 113.03) (width 0.4) (layer B.Cu) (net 14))
 (segment (start 123.19 105.41) (end 125.73 105.41) (width 0.4) (layer B.Cu) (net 13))
 (segment (start 123.19 102.87) (end 125.73 102.87) (width 0.4) (layer B.Cu) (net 12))
 (segment (start 123.19 97.79) (end 125.73 97.79) (width 0.4) (layer B.Cu) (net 11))
 (segment (start 119.38 82.55) (end 125.222 76.708) (width 0.4) (layer B.Cu) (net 15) (status 400000))
 (segment (start 132.588 76.708) (end 135.255 79.375) (width 0.4) (layer B.Cu) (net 15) (status 800000))
 (segment (start 125.222 76.708) (end 132.588 76.708) (width 0.4) (layer B.Cu) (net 15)))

